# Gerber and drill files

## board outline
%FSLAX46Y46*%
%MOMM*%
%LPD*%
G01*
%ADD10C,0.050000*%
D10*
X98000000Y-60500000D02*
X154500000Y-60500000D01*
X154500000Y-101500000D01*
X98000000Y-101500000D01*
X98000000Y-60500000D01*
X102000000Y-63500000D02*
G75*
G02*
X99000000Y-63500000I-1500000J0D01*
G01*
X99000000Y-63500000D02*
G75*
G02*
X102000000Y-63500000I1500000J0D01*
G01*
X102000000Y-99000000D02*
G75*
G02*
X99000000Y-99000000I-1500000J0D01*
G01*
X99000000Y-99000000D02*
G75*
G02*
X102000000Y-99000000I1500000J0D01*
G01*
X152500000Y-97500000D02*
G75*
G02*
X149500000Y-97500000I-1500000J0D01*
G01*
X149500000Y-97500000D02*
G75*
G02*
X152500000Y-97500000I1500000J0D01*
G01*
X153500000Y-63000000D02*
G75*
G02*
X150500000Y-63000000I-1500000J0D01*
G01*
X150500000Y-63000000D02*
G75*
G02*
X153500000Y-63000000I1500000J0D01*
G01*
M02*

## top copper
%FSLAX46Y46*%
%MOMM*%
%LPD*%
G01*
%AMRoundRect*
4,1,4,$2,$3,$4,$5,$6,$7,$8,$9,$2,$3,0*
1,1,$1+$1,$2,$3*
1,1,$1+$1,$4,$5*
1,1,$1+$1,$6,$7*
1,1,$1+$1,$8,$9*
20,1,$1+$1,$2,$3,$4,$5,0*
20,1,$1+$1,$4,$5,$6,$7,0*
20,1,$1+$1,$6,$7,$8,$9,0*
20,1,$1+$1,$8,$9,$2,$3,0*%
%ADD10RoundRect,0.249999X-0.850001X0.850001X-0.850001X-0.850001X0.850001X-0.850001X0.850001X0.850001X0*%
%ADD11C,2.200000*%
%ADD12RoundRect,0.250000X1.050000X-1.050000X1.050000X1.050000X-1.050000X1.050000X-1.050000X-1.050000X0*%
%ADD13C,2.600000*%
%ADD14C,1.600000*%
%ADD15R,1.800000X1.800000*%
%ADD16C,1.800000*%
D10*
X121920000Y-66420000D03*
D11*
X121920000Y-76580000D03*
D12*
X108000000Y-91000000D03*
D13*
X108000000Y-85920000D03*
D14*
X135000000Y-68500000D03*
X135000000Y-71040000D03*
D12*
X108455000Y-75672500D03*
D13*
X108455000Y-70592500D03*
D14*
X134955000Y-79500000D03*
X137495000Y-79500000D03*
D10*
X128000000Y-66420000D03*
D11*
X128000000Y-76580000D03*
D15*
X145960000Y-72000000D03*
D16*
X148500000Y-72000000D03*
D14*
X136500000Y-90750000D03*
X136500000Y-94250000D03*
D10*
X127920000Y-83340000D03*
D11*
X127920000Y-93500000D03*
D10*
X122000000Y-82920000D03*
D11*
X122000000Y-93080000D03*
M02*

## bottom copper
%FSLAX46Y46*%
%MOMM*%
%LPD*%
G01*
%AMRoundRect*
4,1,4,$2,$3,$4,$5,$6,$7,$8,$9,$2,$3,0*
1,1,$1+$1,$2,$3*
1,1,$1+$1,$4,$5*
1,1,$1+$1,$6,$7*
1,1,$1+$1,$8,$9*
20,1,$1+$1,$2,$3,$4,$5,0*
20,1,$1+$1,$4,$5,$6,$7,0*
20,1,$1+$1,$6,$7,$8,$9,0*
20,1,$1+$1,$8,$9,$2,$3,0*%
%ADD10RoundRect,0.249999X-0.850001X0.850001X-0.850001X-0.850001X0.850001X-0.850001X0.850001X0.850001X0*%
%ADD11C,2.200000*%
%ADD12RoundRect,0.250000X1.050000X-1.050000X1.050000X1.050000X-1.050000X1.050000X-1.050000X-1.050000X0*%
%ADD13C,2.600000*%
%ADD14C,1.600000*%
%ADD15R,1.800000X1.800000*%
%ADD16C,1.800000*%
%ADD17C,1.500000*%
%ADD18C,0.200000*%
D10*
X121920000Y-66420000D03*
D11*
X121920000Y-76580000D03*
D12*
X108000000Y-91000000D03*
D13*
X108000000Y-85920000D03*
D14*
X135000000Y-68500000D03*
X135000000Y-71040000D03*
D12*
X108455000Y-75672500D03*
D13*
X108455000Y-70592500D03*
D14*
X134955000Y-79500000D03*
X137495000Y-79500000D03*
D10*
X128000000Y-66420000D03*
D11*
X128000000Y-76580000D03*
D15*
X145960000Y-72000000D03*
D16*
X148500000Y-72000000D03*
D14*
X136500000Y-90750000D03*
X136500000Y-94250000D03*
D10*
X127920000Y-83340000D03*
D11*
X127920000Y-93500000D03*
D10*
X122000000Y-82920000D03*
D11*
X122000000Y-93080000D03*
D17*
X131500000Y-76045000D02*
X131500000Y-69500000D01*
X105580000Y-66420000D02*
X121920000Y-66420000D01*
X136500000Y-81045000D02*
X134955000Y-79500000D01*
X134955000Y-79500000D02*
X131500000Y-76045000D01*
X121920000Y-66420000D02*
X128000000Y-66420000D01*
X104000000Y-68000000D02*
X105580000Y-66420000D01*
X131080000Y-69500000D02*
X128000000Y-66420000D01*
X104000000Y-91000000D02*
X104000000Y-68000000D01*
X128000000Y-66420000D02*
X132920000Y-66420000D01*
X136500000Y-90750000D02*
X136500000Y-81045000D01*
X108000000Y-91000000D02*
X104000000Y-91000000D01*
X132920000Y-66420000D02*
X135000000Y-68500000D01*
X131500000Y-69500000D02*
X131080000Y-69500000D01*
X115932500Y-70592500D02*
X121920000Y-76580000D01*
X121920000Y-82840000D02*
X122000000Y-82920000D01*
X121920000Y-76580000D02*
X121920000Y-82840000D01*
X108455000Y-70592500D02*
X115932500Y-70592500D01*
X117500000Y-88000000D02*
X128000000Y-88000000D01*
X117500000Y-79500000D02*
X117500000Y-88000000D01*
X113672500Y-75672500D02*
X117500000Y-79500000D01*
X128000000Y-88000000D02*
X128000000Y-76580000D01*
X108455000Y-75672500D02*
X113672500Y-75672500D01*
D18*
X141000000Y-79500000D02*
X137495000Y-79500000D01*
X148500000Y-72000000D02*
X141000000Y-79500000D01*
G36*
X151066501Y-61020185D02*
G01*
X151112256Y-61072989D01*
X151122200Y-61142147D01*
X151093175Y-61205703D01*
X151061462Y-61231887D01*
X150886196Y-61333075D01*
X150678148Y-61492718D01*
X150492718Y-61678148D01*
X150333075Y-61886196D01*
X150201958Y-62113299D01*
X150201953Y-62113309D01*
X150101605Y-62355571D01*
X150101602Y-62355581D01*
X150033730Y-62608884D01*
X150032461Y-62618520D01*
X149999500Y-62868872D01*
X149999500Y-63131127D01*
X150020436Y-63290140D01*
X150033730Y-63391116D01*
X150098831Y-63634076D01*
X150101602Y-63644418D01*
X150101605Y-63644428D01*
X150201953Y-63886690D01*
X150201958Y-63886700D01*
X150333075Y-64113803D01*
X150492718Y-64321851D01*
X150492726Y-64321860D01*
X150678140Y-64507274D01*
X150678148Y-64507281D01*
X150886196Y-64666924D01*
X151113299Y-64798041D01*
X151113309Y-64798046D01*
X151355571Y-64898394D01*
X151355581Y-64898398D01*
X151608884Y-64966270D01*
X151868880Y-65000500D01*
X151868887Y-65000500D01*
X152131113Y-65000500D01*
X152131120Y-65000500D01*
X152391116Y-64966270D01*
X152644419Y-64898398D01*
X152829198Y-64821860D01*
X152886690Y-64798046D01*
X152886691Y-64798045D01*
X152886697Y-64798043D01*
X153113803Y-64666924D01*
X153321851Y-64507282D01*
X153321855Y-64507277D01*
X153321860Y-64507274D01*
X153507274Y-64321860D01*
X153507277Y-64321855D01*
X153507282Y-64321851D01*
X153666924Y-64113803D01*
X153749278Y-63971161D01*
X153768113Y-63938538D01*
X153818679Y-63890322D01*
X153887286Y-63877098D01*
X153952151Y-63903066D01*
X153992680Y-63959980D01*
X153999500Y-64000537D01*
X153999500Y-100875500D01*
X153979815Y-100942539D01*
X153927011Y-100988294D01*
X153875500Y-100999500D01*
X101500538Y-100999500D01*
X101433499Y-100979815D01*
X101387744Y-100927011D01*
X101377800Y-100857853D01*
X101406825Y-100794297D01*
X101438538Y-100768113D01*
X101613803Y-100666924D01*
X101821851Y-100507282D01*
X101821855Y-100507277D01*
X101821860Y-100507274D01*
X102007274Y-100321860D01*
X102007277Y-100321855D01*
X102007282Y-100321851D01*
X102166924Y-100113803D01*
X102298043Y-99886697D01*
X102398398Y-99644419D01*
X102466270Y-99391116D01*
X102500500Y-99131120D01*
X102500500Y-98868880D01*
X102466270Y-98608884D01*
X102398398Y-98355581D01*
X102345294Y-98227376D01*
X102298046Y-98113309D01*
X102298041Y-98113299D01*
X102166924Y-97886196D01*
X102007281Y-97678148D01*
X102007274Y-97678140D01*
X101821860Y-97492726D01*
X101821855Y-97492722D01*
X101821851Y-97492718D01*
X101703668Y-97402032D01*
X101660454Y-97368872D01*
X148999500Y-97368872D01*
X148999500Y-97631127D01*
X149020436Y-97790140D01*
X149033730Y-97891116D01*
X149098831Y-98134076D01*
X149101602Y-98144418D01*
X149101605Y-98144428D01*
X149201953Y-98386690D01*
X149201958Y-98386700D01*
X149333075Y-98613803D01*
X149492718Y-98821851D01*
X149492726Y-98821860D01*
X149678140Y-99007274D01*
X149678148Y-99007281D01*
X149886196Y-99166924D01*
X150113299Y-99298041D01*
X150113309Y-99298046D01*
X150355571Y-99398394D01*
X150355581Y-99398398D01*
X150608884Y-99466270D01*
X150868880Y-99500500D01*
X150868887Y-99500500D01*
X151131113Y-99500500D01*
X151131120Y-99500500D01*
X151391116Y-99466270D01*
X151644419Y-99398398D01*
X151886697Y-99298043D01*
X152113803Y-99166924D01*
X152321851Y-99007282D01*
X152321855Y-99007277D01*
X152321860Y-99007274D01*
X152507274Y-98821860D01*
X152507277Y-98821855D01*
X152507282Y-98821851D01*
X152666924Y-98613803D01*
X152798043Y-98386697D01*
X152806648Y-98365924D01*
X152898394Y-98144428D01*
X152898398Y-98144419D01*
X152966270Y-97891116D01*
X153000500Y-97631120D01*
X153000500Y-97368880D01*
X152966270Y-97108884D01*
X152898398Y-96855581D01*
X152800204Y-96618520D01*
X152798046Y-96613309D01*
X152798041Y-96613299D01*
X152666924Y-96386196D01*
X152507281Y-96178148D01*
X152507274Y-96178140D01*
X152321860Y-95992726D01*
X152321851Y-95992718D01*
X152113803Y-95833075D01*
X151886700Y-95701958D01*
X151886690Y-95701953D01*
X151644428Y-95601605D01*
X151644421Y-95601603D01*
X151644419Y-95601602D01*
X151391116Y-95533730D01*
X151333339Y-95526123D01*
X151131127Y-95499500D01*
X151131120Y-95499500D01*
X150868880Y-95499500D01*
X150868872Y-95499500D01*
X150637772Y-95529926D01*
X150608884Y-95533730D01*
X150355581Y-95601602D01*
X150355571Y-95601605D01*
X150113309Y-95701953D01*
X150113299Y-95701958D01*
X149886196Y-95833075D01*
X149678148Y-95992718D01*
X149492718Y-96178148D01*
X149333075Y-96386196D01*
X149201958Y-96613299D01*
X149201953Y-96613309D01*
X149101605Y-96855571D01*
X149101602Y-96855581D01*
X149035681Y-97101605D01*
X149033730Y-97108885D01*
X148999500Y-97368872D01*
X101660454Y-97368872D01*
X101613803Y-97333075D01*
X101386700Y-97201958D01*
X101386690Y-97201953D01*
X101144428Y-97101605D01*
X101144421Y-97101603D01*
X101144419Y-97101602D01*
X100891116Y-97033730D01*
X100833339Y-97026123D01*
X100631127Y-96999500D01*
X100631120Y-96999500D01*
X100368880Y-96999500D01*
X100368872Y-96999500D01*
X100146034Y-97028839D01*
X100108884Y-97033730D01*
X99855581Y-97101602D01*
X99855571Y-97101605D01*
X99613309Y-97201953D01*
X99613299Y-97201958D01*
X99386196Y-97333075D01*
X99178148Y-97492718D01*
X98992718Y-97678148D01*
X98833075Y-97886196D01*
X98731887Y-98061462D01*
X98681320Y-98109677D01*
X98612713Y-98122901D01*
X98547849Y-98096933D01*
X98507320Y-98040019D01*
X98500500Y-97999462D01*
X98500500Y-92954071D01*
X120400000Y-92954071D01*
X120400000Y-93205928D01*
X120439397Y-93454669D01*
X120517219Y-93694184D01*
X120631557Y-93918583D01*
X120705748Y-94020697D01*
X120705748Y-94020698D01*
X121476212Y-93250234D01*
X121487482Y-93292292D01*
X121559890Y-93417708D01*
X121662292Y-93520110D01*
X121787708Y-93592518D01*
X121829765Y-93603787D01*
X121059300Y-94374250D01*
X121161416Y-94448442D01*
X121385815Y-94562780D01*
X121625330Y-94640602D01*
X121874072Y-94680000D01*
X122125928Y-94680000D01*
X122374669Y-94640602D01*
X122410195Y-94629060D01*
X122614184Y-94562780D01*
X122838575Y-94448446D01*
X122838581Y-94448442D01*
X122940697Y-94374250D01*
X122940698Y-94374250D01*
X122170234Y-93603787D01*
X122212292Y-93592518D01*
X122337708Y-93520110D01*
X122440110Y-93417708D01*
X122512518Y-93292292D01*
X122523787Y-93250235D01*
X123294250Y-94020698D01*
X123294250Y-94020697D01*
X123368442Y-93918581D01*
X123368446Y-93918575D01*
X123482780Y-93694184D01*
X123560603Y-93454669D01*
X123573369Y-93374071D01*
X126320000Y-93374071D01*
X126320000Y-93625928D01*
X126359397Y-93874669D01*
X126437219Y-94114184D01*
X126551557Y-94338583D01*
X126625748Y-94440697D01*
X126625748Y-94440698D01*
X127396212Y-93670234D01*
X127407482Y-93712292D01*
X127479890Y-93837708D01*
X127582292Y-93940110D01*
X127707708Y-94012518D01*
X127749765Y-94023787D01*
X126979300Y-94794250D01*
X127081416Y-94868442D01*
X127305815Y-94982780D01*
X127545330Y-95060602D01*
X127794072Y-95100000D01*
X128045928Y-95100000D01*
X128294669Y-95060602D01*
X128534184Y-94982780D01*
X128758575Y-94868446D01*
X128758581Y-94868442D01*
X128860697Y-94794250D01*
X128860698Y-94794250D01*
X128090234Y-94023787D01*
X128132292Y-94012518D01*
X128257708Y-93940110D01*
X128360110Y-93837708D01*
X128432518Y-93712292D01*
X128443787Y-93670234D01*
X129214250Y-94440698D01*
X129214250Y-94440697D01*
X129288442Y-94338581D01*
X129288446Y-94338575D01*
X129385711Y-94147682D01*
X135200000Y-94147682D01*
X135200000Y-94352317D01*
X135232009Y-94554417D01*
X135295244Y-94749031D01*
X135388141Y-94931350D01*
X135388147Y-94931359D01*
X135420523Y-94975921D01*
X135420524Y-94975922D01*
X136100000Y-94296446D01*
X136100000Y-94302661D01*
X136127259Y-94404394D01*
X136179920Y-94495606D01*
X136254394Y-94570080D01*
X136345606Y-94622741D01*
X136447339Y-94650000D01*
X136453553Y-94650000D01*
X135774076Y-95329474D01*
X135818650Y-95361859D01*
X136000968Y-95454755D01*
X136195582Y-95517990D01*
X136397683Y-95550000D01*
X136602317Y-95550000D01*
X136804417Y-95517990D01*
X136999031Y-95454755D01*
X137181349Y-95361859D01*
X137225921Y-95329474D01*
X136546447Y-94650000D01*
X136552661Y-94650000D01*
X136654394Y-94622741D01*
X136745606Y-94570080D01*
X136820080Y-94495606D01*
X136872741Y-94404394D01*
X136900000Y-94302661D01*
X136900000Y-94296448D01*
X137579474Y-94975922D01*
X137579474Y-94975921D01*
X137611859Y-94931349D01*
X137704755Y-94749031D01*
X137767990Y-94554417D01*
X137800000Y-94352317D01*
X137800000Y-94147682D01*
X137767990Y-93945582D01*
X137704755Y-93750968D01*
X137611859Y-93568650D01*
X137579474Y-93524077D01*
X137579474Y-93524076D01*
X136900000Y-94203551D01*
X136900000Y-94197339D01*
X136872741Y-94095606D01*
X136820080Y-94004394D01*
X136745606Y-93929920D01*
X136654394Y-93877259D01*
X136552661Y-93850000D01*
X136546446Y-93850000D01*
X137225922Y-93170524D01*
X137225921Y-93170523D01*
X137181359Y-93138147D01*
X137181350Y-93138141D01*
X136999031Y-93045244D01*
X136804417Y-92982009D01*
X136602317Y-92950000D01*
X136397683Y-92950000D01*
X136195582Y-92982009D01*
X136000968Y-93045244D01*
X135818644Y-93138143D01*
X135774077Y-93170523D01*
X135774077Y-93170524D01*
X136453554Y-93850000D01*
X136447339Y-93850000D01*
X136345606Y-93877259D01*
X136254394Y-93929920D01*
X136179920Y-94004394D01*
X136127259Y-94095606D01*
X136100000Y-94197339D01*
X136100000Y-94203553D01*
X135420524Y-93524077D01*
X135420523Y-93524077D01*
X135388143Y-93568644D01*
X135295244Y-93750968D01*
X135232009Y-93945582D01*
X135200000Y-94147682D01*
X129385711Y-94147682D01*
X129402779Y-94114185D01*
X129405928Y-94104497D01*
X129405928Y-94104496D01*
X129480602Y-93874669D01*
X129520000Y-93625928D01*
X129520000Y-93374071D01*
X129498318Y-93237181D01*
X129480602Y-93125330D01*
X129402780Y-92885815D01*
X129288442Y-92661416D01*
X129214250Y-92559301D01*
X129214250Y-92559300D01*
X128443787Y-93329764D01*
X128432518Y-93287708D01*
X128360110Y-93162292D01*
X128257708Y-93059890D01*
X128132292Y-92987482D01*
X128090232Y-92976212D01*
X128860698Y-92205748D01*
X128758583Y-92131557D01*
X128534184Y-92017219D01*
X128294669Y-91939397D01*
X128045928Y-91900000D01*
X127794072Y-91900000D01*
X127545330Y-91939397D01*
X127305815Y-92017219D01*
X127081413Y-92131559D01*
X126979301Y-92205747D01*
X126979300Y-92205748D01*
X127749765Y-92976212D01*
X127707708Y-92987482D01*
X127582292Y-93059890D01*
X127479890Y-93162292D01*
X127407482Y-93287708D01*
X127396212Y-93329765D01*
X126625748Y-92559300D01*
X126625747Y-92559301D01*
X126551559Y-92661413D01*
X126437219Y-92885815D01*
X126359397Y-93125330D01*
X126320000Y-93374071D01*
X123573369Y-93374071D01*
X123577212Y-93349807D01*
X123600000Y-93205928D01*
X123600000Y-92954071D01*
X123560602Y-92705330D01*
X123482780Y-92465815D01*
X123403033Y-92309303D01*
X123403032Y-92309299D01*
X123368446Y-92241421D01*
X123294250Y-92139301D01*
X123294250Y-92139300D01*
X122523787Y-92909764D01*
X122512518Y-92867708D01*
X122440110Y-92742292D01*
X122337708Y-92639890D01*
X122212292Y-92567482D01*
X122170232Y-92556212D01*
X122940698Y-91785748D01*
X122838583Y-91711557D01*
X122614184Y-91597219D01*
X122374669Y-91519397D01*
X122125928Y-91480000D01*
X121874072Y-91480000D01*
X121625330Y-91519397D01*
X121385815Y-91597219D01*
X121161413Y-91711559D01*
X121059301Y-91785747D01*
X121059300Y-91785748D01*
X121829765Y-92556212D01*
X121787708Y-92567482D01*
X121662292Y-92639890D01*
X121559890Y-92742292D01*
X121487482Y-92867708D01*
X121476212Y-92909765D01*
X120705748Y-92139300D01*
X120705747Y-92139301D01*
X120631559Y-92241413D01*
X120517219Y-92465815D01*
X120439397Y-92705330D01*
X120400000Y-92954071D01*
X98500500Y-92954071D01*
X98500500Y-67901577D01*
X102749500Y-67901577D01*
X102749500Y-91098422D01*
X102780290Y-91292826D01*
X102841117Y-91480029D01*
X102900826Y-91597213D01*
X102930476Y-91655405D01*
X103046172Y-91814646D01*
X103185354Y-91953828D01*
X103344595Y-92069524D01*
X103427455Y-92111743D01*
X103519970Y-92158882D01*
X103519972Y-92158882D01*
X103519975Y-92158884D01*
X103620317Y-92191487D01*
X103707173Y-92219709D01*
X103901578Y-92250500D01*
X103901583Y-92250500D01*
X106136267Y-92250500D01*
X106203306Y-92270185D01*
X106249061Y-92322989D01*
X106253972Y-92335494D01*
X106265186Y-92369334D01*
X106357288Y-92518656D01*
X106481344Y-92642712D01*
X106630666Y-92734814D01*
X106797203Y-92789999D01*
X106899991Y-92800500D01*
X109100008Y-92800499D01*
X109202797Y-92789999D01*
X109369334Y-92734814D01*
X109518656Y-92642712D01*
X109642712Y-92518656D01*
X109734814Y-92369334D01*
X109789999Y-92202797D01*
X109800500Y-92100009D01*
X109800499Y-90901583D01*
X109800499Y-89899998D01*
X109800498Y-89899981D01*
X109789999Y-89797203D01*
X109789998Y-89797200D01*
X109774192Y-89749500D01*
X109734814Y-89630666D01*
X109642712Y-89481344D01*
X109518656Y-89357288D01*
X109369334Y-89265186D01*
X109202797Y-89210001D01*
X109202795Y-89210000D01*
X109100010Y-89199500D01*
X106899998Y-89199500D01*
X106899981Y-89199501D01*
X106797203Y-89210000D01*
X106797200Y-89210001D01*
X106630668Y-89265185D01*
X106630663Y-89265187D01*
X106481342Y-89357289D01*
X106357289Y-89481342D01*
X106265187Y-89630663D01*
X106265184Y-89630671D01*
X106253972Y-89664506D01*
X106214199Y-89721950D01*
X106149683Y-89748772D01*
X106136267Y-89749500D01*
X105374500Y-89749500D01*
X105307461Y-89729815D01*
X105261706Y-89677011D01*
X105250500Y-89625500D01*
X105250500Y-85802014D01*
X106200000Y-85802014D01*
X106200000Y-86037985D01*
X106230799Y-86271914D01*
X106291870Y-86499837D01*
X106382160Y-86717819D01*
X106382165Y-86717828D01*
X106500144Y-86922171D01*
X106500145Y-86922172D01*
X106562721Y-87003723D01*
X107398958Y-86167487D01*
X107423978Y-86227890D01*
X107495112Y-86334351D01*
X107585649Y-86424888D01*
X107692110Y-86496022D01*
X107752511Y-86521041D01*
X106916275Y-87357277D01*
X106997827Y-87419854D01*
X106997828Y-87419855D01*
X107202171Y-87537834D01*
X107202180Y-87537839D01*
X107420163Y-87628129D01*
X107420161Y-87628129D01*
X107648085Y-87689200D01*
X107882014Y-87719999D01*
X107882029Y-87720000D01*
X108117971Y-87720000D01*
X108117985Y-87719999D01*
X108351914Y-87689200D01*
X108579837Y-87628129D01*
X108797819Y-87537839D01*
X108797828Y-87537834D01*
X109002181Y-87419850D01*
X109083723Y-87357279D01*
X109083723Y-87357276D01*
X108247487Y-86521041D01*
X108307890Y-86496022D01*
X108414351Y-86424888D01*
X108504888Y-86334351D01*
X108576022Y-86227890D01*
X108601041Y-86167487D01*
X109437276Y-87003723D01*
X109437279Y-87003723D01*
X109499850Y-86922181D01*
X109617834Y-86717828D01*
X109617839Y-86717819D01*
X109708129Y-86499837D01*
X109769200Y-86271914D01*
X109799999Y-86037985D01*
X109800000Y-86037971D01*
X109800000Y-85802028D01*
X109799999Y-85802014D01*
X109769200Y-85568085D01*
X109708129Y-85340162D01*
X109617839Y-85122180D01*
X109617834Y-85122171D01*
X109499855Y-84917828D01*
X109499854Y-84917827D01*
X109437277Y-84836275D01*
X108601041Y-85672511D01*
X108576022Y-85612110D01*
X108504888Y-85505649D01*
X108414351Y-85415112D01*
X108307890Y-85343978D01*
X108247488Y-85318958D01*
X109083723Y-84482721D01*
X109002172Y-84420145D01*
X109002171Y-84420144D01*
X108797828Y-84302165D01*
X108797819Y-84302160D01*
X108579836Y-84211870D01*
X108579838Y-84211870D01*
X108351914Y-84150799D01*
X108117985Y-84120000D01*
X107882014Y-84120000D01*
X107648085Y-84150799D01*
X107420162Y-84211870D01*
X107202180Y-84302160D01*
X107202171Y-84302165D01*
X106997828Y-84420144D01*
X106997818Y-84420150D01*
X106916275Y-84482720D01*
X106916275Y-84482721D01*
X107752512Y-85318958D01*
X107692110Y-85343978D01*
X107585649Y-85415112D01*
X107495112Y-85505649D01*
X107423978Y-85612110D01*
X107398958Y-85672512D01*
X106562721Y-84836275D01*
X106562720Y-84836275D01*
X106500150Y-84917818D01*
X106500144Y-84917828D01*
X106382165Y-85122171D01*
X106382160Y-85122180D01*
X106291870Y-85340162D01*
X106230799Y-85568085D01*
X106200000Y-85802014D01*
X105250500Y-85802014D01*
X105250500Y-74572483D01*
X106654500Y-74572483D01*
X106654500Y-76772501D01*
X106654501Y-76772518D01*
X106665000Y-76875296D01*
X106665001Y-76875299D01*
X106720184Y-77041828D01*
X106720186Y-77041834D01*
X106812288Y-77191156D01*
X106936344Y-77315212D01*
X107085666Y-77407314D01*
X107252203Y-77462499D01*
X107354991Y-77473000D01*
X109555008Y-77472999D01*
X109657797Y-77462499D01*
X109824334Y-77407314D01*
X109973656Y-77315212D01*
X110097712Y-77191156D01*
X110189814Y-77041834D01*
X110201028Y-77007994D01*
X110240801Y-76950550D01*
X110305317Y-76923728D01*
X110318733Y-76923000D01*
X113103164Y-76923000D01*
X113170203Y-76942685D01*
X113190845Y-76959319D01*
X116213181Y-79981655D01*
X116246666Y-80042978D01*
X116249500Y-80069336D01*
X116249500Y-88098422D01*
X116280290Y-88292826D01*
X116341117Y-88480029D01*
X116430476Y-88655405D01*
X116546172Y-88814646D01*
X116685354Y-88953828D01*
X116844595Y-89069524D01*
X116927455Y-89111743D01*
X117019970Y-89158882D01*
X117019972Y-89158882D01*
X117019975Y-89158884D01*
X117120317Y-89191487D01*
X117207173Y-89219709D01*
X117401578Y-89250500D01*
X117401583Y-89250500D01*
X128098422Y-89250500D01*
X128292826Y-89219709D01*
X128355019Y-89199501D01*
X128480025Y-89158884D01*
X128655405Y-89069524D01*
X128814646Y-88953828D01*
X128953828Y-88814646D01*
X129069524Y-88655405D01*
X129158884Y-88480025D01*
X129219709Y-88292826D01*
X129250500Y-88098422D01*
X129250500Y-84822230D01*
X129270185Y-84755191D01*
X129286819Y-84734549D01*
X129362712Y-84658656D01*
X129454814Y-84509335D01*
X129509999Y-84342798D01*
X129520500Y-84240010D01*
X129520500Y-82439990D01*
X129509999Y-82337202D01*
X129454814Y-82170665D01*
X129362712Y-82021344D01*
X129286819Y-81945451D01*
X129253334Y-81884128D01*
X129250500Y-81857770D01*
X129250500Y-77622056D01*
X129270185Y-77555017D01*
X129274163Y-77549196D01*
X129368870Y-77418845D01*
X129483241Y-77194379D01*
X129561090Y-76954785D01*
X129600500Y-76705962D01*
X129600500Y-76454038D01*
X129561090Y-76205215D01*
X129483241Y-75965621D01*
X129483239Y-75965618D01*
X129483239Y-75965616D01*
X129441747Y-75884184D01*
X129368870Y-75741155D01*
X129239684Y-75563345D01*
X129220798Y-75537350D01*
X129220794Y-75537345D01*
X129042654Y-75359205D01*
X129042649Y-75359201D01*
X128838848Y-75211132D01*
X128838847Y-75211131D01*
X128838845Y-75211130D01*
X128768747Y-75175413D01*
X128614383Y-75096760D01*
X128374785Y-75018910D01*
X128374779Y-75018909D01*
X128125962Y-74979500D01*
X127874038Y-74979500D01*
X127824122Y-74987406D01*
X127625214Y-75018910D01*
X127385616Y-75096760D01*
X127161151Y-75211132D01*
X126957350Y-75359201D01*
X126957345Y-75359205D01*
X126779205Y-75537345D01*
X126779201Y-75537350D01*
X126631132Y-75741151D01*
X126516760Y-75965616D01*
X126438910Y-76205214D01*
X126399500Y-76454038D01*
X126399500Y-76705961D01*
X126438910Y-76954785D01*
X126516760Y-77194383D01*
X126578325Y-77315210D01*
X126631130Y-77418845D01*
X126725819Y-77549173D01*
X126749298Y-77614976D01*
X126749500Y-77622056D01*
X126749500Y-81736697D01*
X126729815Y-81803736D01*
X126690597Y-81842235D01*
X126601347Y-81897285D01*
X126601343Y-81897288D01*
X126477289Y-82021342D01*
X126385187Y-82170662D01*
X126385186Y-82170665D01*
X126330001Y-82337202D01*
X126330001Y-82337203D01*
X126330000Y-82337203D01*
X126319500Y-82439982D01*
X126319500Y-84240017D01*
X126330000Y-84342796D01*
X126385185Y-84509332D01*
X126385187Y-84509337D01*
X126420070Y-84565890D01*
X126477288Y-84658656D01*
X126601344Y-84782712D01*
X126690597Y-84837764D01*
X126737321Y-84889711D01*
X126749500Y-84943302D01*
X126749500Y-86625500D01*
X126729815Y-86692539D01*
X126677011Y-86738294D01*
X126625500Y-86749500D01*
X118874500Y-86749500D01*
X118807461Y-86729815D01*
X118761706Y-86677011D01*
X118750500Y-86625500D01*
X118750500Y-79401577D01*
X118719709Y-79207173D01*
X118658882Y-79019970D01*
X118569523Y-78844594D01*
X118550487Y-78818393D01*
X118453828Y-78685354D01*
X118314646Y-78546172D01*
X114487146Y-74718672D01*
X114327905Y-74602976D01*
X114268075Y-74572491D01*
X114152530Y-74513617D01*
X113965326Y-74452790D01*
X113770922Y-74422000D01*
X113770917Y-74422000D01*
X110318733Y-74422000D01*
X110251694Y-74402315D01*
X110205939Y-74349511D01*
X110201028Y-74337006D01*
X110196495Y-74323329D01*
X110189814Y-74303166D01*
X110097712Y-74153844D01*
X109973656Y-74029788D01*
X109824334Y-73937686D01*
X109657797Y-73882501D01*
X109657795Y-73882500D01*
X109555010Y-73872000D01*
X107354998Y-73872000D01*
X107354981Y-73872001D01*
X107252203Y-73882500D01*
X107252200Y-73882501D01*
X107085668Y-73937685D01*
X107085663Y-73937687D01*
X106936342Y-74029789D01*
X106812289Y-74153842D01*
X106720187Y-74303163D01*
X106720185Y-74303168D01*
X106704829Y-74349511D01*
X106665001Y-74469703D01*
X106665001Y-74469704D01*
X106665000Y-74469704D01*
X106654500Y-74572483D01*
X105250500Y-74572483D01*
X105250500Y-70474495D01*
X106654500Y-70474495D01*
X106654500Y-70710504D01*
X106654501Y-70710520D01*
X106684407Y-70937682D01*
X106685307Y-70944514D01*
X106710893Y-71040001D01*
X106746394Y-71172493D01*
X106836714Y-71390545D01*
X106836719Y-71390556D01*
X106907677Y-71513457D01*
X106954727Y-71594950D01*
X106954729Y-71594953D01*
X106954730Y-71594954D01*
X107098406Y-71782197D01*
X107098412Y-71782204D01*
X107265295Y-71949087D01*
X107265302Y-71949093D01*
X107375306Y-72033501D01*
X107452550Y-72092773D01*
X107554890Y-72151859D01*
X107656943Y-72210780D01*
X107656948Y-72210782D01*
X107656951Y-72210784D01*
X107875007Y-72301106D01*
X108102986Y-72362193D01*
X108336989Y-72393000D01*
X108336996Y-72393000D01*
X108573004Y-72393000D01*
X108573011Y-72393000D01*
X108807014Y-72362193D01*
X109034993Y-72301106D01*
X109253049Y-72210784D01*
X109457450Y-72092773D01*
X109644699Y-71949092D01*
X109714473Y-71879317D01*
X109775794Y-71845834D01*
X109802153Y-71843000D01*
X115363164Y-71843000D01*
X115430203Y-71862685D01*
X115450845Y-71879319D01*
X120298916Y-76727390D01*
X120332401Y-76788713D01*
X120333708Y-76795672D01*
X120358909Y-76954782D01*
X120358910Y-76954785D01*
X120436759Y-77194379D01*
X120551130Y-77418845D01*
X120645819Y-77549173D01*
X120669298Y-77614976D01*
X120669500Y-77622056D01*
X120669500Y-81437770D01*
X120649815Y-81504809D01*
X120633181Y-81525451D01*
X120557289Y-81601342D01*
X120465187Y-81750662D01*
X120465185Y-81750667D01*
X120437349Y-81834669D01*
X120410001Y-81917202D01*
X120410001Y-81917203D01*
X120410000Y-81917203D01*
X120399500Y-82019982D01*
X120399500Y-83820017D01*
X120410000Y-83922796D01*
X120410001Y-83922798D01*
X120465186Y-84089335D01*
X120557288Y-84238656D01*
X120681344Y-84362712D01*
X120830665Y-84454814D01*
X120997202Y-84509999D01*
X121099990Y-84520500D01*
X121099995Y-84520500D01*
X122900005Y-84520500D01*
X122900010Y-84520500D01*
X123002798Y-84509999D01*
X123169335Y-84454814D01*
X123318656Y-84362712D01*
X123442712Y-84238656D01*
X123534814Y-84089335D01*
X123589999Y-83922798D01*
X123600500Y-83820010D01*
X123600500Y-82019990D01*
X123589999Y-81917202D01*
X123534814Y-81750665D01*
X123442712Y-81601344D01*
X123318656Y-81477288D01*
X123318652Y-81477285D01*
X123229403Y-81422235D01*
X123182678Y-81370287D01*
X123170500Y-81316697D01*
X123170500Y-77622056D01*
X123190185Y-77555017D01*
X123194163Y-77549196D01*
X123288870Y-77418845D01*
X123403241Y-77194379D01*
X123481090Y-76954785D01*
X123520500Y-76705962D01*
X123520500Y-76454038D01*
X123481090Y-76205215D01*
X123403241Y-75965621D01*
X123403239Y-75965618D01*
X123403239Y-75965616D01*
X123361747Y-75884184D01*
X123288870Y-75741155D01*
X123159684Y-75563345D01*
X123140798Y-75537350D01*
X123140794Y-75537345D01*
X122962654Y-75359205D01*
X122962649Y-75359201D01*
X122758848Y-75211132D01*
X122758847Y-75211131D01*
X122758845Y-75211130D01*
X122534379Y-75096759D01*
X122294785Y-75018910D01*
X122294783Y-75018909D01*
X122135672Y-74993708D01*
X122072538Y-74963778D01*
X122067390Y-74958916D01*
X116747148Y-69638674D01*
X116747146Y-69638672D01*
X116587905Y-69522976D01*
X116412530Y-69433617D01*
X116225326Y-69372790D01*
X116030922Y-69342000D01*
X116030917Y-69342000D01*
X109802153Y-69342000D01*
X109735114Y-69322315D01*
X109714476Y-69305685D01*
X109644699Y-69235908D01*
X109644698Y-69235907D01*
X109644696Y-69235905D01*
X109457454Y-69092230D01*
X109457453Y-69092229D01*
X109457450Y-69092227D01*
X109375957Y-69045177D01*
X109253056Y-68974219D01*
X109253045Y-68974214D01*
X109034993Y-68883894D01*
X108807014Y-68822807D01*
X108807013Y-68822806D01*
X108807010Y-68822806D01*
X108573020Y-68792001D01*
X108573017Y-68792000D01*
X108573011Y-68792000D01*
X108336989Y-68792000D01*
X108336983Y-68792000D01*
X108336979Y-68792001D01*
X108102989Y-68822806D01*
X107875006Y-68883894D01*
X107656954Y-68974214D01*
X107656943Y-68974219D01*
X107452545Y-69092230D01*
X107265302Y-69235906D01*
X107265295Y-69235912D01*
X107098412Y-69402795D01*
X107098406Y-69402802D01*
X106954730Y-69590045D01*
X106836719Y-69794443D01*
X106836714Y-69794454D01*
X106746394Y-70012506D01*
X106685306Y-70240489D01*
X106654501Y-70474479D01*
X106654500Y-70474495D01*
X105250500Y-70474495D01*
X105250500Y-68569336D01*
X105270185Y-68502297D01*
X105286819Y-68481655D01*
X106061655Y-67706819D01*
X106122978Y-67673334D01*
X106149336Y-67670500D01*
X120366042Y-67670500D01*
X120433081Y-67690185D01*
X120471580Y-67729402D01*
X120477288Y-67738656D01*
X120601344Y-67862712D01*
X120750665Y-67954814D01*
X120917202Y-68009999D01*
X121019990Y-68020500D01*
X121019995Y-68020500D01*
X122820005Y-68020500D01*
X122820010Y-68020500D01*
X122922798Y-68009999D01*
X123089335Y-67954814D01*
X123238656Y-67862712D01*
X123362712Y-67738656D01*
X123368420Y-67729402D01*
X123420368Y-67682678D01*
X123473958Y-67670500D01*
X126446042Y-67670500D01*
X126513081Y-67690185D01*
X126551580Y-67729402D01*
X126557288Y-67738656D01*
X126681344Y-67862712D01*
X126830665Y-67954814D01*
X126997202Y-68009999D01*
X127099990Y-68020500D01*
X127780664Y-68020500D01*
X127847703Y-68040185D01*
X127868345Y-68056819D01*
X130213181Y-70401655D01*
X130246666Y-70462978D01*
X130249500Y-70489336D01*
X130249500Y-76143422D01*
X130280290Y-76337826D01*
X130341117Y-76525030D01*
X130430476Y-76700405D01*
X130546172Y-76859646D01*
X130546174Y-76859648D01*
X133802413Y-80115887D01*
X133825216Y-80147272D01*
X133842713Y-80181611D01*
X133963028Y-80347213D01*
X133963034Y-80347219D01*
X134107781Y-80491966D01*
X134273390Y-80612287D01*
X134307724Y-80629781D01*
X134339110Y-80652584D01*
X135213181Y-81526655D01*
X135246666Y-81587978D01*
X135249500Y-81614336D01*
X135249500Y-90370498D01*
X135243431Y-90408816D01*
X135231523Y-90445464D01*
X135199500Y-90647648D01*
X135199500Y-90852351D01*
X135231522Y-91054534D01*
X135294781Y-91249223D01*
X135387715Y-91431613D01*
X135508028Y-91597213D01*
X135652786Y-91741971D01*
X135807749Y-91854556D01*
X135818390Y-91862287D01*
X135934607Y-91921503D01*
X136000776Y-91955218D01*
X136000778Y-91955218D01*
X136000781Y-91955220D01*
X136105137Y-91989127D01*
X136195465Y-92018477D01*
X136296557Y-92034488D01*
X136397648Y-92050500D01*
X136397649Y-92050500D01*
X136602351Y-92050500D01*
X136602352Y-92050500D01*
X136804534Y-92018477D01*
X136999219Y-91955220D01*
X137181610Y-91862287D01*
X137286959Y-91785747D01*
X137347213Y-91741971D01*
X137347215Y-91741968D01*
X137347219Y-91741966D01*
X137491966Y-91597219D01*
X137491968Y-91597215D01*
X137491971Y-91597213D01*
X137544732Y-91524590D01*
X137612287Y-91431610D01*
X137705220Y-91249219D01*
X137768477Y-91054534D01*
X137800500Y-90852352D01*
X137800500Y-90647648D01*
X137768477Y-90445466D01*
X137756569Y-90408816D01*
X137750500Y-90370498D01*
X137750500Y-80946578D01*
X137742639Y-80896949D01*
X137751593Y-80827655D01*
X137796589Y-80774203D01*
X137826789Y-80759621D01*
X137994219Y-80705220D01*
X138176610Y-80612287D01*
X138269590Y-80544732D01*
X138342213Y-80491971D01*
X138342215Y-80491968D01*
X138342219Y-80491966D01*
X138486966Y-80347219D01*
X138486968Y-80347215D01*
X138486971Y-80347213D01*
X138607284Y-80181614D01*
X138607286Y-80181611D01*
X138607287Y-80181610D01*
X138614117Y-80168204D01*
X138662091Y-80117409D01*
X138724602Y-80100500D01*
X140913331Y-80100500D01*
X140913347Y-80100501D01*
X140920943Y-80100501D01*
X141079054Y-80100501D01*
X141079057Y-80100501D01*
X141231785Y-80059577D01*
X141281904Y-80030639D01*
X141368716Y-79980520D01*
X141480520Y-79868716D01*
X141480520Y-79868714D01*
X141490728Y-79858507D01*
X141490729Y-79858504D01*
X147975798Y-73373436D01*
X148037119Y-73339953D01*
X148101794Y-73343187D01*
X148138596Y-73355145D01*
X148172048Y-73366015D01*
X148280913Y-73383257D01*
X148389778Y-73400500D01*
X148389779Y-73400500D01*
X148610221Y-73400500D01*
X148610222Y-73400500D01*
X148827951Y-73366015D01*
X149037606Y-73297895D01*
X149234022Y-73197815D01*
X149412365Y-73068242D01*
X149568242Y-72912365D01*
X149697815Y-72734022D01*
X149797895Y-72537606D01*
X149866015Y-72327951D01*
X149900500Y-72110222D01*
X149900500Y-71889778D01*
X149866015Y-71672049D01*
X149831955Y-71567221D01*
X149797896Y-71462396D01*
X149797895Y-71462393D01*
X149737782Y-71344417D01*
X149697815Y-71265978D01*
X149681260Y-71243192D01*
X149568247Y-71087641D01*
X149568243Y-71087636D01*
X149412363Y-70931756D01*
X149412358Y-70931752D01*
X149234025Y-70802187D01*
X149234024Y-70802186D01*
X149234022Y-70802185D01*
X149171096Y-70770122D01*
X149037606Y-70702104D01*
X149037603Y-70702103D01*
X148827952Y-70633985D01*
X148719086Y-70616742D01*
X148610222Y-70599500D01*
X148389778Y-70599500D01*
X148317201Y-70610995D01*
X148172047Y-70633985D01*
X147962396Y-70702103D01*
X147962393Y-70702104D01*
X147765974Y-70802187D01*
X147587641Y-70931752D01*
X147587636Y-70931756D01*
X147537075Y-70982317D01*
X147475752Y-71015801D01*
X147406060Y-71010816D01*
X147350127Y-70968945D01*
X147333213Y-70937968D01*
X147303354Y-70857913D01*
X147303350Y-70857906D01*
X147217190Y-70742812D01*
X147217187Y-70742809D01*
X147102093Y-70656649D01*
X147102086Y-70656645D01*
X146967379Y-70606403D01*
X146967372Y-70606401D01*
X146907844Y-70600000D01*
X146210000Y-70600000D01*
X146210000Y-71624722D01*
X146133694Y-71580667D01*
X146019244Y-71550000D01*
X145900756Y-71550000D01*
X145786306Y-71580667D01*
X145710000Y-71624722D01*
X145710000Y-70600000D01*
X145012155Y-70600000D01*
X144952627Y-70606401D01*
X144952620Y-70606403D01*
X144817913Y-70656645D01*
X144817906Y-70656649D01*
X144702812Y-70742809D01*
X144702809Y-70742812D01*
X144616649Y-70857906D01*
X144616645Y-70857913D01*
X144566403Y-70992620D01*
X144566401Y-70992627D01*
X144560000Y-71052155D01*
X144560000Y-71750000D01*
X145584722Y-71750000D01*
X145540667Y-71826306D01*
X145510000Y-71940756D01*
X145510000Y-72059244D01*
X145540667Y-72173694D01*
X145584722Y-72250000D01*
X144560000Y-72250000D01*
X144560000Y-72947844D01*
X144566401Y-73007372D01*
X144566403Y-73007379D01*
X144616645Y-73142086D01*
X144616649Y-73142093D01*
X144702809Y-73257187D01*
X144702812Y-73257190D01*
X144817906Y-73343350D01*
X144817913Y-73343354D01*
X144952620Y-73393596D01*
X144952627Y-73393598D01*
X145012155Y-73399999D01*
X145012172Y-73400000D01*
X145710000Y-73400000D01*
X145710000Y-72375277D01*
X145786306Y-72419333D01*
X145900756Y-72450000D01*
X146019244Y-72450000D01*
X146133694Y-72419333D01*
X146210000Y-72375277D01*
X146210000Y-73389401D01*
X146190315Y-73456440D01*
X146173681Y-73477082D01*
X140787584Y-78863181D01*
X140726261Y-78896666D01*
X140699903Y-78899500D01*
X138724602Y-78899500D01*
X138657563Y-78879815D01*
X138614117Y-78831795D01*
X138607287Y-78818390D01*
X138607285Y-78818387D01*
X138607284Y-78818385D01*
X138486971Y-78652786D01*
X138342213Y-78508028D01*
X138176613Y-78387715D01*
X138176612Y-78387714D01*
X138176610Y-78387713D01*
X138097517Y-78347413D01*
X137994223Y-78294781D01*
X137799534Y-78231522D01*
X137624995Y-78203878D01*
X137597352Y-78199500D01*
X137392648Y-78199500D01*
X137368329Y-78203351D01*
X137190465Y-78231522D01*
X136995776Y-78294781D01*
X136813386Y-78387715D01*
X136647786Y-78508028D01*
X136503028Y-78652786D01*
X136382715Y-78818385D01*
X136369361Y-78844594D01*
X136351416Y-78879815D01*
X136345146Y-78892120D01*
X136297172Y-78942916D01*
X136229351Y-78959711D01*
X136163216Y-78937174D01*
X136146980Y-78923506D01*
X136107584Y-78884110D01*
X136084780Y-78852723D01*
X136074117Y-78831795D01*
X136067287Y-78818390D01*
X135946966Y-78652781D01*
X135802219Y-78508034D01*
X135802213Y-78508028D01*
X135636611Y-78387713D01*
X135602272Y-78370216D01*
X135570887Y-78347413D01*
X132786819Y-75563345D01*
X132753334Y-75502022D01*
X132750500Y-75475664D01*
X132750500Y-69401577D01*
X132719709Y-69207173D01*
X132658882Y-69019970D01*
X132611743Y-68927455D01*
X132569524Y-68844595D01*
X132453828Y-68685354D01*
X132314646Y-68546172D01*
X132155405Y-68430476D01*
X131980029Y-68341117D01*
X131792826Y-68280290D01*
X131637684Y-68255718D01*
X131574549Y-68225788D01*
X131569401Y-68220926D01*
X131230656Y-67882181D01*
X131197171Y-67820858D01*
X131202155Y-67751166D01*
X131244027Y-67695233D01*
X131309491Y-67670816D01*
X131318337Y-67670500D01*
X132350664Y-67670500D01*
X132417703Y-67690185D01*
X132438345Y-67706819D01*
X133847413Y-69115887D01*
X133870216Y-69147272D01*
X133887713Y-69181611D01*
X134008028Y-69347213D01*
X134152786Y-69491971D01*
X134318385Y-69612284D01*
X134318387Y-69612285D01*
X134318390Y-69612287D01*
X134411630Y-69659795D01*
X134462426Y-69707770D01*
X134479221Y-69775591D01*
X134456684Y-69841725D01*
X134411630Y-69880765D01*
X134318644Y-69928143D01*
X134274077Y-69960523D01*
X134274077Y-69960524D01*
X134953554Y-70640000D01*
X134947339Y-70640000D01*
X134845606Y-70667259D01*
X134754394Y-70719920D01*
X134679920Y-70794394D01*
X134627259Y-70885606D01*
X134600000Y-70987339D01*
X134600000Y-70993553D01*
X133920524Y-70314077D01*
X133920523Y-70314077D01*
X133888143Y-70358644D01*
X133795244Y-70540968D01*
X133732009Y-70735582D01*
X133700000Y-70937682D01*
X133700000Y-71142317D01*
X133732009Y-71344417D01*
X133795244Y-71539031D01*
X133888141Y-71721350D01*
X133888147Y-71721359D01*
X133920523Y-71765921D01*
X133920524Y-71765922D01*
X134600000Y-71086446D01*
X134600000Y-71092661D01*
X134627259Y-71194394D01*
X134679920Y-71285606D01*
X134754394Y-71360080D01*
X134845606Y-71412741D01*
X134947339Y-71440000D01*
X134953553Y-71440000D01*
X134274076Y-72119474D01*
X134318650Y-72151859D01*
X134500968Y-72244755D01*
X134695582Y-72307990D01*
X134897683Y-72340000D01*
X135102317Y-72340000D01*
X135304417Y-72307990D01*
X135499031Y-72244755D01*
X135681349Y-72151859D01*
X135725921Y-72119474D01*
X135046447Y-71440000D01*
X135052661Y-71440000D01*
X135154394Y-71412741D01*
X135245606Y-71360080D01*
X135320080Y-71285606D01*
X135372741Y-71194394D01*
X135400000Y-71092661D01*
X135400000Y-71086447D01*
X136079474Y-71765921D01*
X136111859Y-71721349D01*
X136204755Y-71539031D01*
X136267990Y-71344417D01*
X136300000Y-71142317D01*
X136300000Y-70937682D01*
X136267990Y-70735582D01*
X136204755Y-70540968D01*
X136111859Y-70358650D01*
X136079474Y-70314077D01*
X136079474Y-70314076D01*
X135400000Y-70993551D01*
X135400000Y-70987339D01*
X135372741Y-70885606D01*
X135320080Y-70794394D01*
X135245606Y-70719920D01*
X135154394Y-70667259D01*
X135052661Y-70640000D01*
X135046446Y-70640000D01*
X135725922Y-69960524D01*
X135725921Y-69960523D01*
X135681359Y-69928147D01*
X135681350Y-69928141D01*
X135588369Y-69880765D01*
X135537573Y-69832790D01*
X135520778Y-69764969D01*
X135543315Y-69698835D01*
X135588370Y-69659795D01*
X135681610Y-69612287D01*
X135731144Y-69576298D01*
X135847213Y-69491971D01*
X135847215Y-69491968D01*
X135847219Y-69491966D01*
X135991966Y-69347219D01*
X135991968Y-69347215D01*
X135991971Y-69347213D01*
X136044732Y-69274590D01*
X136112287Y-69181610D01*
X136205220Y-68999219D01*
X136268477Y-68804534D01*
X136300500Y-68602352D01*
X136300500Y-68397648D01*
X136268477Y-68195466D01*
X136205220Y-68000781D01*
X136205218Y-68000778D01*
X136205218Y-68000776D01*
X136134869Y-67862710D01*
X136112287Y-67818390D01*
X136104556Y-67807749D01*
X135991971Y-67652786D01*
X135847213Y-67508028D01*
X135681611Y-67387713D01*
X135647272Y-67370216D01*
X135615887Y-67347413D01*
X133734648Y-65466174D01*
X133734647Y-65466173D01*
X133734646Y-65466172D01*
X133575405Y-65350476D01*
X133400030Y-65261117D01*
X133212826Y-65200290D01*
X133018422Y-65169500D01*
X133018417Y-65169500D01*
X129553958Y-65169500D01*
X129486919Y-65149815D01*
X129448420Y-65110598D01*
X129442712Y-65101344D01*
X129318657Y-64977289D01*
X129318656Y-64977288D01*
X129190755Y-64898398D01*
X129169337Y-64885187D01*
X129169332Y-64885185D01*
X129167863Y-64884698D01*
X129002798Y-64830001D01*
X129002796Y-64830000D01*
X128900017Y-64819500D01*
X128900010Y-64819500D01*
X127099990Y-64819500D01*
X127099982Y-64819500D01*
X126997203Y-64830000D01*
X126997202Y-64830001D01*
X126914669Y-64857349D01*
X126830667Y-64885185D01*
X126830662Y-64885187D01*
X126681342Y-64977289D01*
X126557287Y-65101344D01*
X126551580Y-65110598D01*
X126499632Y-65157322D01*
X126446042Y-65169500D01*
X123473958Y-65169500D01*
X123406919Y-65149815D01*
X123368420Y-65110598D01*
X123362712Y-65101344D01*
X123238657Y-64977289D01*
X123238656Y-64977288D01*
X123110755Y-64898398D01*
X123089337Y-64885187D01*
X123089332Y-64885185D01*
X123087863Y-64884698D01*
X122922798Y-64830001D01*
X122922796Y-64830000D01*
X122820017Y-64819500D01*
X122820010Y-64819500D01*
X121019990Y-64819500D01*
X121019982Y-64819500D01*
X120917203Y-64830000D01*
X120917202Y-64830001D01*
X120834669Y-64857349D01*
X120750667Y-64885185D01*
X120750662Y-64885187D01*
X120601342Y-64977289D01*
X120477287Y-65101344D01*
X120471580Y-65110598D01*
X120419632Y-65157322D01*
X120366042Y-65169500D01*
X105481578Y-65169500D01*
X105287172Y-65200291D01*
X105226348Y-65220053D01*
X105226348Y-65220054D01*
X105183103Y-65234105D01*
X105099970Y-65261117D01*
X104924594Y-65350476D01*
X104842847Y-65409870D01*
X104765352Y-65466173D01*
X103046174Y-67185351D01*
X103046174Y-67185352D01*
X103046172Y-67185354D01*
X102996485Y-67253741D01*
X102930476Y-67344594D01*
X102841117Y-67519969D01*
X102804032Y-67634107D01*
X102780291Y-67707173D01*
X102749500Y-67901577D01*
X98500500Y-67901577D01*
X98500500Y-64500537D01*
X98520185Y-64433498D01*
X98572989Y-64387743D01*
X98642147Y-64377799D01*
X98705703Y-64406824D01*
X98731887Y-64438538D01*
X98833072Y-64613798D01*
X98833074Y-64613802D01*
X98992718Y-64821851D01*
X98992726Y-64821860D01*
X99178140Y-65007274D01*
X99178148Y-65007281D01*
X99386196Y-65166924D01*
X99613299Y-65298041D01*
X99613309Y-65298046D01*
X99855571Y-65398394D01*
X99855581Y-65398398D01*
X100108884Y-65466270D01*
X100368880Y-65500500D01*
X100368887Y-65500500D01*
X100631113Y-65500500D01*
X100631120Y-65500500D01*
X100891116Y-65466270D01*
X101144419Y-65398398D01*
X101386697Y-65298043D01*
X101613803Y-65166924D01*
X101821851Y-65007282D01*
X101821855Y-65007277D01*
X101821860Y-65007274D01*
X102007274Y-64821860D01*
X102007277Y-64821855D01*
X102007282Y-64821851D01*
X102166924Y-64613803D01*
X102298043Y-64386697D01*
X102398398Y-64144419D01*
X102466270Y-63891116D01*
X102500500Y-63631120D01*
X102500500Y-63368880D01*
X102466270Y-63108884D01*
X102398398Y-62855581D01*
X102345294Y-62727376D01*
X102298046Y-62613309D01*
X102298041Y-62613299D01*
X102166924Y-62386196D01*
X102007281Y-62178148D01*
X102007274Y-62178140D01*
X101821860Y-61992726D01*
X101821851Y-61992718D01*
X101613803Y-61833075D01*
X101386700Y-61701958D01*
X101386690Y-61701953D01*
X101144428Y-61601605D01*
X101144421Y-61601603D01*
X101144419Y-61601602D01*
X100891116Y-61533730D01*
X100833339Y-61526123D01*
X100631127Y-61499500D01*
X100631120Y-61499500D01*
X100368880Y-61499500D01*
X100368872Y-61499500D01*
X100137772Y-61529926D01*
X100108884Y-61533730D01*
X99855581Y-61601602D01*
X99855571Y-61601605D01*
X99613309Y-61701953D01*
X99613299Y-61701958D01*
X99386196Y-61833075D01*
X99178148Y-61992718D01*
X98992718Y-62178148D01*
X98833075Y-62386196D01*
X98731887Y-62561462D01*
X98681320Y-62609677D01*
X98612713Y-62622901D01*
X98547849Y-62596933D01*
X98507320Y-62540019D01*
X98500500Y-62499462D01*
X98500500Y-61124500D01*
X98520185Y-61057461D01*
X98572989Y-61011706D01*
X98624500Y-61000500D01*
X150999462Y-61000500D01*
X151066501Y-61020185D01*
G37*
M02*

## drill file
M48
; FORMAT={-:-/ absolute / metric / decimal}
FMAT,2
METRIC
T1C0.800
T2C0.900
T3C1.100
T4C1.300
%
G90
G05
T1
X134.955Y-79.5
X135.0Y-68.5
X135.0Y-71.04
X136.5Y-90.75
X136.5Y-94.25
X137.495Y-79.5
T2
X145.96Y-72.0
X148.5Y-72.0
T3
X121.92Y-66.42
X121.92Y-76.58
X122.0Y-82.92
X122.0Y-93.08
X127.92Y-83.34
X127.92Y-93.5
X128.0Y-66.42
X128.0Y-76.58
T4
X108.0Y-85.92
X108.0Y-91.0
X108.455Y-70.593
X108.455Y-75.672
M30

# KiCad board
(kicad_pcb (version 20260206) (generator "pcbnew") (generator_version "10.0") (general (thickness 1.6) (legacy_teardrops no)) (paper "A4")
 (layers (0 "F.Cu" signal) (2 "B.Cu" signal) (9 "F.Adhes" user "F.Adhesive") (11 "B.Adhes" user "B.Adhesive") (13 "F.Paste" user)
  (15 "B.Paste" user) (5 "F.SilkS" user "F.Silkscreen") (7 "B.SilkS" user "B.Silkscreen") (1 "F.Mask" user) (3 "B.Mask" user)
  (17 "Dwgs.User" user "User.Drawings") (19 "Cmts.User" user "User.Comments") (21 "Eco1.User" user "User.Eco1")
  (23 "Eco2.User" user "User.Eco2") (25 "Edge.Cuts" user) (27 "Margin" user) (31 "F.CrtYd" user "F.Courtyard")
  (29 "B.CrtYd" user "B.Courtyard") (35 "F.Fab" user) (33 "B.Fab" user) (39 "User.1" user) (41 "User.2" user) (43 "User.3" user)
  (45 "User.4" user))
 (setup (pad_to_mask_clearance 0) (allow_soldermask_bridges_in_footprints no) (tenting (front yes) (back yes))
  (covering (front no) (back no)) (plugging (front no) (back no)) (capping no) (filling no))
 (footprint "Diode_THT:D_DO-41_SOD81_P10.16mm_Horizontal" (layer "F.Cu") (at 121.92 66.42 -90)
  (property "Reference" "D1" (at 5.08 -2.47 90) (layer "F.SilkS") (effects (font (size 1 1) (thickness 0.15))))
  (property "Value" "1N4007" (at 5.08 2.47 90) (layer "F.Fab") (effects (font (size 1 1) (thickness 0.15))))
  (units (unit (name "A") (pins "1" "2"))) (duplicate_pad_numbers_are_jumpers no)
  (pad "1" thru_hole roundrect (at 0 0 270) (size 2.2 2.2) (drill 1.1) (layers "*.Cu" "*.Mask") (remove_unused_layers no)
   (roundrect_rratio 0.113636) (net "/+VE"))
  (pad "2" thru_hole circle (at 10.16 0 270) (size 2.2 2.2) (drill 1.1) (layers "*.Cu" "*.Mask") (remove_unused_layers no)
   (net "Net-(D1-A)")))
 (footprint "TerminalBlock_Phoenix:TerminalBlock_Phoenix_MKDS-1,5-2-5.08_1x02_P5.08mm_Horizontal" (layer "F.Cu") (at 108 91 90)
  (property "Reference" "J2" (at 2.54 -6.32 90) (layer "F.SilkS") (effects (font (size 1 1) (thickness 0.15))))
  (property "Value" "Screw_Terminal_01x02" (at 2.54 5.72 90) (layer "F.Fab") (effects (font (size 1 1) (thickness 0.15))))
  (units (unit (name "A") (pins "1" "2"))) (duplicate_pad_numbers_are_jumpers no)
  (pad "1" thru_hole roundrect (at 0 0 90) (size 2.6 2.6) (drill 1.3) (layers "*.Cu" "*.Mask") (remove_unused_layers no)
   (roundrect_rratio 0.096154) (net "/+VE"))
  (pad "2" thru_hole circle (at 5.08 0 90) (size 2.6 2.6) (drill 1.3) (layers "*.Cu" "*.Mask") (remove_unused_layers no) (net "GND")))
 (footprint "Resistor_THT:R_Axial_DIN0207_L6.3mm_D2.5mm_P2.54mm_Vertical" (layer "F.Cu") (at 135 68.5 -90)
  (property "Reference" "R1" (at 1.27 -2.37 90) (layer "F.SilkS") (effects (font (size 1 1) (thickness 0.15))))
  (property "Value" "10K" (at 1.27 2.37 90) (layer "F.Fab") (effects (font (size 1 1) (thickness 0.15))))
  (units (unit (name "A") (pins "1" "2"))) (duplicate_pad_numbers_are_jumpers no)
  (pad "1" thru_hole circle (at 0 0 270) (size 1.6 1.6) (drill 0.8) (layers "*.Cu" "*.Mask") (remove_unused_layers no) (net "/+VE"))
  (pad "2" thru_hole circle (at 2.54 0 270) (size 1.6 1.6) (drill 0.8) (layers "*.Cu" "*.Mask") (remove_unused_layers no) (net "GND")))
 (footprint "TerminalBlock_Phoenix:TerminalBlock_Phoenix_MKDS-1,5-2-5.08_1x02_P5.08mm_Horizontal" (layer "F.Cu") (at 108.455 75.6725 90)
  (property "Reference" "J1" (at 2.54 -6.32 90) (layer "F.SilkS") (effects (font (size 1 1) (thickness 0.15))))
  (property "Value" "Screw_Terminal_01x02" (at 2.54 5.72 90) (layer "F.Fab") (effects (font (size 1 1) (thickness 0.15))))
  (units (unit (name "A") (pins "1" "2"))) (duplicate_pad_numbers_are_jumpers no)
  (pad "1" thru_hole roundrect (at 0 0 90) (size 2.6 2.6) (drill 1.3) (layers "*.Cu" "*.Mask") (remove_unused_layers no)
   (roundrect_rratio 0.096154) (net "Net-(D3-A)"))
  (pad "2" thru_hole circle (at 5.08 0 90) (size 2.6 2.6) (drill 1.3) (layers "*.Cu" "*.Mask") (remove_unused_layers no) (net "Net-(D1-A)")))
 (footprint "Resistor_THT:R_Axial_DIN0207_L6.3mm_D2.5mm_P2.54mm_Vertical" (layer "F.Cu") (at 134.955 79.5)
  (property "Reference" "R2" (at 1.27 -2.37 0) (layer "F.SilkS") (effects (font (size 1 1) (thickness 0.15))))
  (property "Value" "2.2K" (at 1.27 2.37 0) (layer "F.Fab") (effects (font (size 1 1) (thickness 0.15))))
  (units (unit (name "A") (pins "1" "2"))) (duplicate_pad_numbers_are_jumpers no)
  (pad "1" thru_hole circle (at 0 0) (size 1.6 1.6) (drill 0.8) (layers "*.Cu" "*.Mask") (remove_unused_layers no) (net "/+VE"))
  (pad "2" thru_hole circle (at 2.54 0) (size 1.6 1.6) (drill 0.8) (layers "*.Cu" "*.Mask") (remove_unused_layers no) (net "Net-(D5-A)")))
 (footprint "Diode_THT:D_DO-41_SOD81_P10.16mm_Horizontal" (layer "F.Cu") (at 128 66.42 -90)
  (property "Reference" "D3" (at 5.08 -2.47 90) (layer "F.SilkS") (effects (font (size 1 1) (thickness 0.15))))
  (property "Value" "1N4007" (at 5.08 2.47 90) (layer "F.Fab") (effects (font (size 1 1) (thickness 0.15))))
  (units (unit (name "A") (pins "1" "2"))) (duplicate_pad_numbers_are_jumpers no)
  (pad "1" thru_hole roundrect (at 0 0 270) (size 2.2 2.2) (drill 1.1) (layers "*.Cu" "*.Mask") (remove_unused_layers no)
   (roundrect_rratio 0.113636) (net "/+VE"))
  (pad "2" thru_hole circle (at 10.16 0 270) (size 2.2 2.2) (drill 1.1) (layers "*.Cu" "*.Mask") (remove_unused_layers no)
   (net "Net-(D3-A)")))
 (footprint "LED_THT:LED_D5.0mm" (layer "F.Cu") (at 145.96 72)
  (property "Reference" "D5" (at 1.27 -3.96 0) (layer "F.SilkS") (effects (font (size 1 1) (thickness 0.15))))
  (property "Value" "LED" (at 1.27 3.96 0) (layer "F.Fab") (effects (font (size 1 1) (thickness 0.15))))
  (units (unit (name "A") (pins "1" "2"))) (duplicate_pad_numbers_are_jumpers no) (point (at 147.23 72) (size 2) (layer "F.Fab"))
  (pad "1" thru_hole rect (at 0 0) (size 1.8 1.8) (drill 0.9) (layers "*.Cu" "*.Mask") (remove_unused_layers no) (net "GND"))
  (pad "2" thru_hole circle (at 2.54 0) (size 1.8 1.8) (drill 0.9) (layers "*.Cu" "*.Mask") (remove_unused_layers no) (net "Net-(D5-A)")))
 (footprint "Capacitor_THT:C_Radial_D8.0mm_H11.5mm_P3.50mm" (layer "F.Cu") (at 136.5 90.75 -90)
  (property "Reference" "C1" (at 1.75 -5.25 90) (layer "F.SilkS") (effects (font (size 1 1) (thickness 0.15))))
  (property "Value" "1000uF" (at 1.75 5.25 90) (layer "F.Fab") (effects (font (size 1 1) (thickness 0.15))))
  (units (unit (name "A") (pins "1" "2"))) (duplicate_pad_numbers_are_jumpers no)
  (pad "1" thru_hole circle (at 0 0 270) (size 1.6 1.6) (drill 0.8) (layers "*.Cu" "*.Mask") (remove_unused_layers no) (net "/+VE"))
  (pad "2" thru_hole circle (at 3.5 0 270) (size 1.6 1.6) (drill 0.8) (layers "*.Cu" "*.Mask") (remove_unused_layers no) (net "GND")))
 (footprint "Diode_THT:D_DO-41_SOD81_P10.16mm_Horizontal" (layer "F.Cu") (at 127.92 83.34 -90)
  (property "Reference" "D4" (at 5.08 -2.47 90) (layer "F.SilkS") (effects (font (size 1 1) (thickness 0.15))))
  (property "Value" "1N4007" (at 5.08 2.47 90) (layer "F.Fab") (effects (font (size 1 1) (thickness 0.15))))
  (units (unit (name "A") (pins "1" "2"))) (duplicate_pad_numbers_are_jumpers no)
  (pad "1" thru_hole roundrect (at 0 0 270) (size 2.2 2.2) (drill 1.1) (layers "*.Cu" "*.Mask") (remove_unused_layers no)
   (roundrect_rratio 0.113636) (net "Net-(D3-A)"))
  (pad "2" thru_hole circle (at 10.16 0 270) (size 2.2 2.2) (drill 1.1) (layers "*.Cu" "*.Mask") (remove_unused_layers no) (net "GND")))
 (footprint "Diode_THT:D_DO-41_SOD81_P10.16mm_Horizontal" (layer "F.Cu") (at 122 82.92 -90)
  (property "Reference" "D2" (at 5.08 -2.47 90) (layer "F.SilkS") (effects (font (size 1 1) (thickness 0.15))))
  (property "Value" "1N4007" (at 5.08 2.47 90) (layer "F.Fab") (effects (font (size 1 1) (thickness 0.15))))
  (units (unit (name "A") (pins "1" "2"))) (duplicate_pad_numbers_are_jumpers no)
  (pad "1" thru_hole roundrect (at 0 0 270) (size 2.2 2.2) (drill 1.1) (layers "*.Cu" "*.Mask") (remove_unused_layers no)
   (roundrect_rratio 0.113636) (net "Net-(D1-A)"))
  (pad "2" thru_hole circle (at 10.16 0 270) (size 2.2 2.2) (drill 1.1) (layers "*.Cu" "*.Mask") (remove_unused_layers no) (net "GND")))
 (gr_rect (start 98 60.5) (end 154.5 101.5) (stroke (width 0.05) (type default)) (fill no) (layer "Edge.Cuts"))
 (gr_circle (center 100.5 63.5) (end 102 63.5) (stroke (width 0.05) (type default)) (fill no) (layer "Edge.Cuts"))
 (gr_circle (center 100.5 99) (end 102 99) (stroke (width 0.05) (type default)) (fill no) (layer "Edge.Cuts"))
 (gr_circle (center 151 97.5) (end 152.5 97.5) (stroke (width 0.05) (type default)) (fill no) (layer "Edge.Cuts"))
 (gr_circle (center 152 63) (end 153.5 63) (stroke (width 0.05) (type default)) (fill no) (layer "Edge.Cuts"))
 (segment (start 131.5 76.045) (end 131.5 69.5) (width 1.5) (layer "B.Cu") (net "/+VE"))
 (segment (start 105.58 66.42) (end 121.92 66.42) (width 1.5) (layer "B.Cu") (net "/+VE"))
 (segment (start 136.5 81.045) (end 134.955 79.5) (width 1.5) (layer "B.Cu") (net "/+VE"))
 (segment (start 134.955 79.5) (end 131.5 76.045) (width 1.5) (layer "B.Cu") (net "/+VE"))
 (segment (start 121.92 66.42) (end 128 66.42) (width 1.5) (layer "B.Cu") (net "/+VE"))
 (segment (start 104 68) (end 105.58 66.42) (width 1.5) (layer "B.Cu") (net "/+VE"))
 (segment (start 131.08 69.5) (end 128 66.42) (width 1.5) (layer "B.Cu") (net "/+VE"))
 (segment (start 104 91) (end 104 68) (width 1.5) (layer "B.Cu") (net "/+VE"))
 (segment (start 128 66.42) (end 132.92 66.42) (width 1.5) (layer "B.Cu") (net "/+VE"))
 (segment (start 136.5 90.75) (end 136.5 81.045) (width 1.5) (layer "B.Cu") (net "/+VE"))
 (segment (start 108 91) (end 104 91) (width 1.5) (layer "B.Cu") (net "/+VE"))
 (segment (start 132.92 66.42) (end 135 68.5) (width 1.5) (layer "B.Cu") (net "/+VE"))
 (segment (start 131.5 69.5) (end 131.08 69.5) (width 1.5) (layer "B.Cu") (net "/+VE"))
 (segment (start 115.9325 70.5925) (end 121.92 76.58) (width 1.5) (layer "B.Cu") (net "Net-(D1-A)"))
 (segment (start 121.92 82.84) (end 122 82.92) (width 1.5) (layer "B.Cu") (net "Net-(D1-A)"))
 (segment (start 121.92 76.58) (end 121.92 82.84) (width 1.5) (layer "B.Cu") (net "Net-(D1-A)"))
 (segment (start 108.455 70.5925) (end 115.9325 70.5925) (width 1.5) (layer "B.Cu") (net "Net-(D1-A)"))
 (segment (start 117.5 88) (end 128 88) (width 1.5) (layer "B.Cu") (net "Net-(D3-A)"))
 (segment (start 117.5 79.5) (end 117.5 88) (width 1.5) (layer "B.Cu") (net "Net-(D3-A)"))
 (segment (start 113.6725 75.6725) (end 117.5 79.5) (width 1.5) (layer "B.Cu") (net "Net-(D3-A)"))
 (segment (start 128 88) (end 128 76.58) (width 1.5) (layer "B.Cu") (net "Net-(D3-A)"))
 (segment (start 108.455 75.6725) (end 113.6725 75.6725) (width 1.5) (layer "B.Cu") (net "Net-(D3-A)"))
 (segment (start 141 79.5) (end 137.495 79.5) (width 0.2) (layer "B.Cu") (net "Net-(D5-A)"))
 (segment (start 148.5 72) (end 141 79.5) (width 0.2) (layer "B.Cu") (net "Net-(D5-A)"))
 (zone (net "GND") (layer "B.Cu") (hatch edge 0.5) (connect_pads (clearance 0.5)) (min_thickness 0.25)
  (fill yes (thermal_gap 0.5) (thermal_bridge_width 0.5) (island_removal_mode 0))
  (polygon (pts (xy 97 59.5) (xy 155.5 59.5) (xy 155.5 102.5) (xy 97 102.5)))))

